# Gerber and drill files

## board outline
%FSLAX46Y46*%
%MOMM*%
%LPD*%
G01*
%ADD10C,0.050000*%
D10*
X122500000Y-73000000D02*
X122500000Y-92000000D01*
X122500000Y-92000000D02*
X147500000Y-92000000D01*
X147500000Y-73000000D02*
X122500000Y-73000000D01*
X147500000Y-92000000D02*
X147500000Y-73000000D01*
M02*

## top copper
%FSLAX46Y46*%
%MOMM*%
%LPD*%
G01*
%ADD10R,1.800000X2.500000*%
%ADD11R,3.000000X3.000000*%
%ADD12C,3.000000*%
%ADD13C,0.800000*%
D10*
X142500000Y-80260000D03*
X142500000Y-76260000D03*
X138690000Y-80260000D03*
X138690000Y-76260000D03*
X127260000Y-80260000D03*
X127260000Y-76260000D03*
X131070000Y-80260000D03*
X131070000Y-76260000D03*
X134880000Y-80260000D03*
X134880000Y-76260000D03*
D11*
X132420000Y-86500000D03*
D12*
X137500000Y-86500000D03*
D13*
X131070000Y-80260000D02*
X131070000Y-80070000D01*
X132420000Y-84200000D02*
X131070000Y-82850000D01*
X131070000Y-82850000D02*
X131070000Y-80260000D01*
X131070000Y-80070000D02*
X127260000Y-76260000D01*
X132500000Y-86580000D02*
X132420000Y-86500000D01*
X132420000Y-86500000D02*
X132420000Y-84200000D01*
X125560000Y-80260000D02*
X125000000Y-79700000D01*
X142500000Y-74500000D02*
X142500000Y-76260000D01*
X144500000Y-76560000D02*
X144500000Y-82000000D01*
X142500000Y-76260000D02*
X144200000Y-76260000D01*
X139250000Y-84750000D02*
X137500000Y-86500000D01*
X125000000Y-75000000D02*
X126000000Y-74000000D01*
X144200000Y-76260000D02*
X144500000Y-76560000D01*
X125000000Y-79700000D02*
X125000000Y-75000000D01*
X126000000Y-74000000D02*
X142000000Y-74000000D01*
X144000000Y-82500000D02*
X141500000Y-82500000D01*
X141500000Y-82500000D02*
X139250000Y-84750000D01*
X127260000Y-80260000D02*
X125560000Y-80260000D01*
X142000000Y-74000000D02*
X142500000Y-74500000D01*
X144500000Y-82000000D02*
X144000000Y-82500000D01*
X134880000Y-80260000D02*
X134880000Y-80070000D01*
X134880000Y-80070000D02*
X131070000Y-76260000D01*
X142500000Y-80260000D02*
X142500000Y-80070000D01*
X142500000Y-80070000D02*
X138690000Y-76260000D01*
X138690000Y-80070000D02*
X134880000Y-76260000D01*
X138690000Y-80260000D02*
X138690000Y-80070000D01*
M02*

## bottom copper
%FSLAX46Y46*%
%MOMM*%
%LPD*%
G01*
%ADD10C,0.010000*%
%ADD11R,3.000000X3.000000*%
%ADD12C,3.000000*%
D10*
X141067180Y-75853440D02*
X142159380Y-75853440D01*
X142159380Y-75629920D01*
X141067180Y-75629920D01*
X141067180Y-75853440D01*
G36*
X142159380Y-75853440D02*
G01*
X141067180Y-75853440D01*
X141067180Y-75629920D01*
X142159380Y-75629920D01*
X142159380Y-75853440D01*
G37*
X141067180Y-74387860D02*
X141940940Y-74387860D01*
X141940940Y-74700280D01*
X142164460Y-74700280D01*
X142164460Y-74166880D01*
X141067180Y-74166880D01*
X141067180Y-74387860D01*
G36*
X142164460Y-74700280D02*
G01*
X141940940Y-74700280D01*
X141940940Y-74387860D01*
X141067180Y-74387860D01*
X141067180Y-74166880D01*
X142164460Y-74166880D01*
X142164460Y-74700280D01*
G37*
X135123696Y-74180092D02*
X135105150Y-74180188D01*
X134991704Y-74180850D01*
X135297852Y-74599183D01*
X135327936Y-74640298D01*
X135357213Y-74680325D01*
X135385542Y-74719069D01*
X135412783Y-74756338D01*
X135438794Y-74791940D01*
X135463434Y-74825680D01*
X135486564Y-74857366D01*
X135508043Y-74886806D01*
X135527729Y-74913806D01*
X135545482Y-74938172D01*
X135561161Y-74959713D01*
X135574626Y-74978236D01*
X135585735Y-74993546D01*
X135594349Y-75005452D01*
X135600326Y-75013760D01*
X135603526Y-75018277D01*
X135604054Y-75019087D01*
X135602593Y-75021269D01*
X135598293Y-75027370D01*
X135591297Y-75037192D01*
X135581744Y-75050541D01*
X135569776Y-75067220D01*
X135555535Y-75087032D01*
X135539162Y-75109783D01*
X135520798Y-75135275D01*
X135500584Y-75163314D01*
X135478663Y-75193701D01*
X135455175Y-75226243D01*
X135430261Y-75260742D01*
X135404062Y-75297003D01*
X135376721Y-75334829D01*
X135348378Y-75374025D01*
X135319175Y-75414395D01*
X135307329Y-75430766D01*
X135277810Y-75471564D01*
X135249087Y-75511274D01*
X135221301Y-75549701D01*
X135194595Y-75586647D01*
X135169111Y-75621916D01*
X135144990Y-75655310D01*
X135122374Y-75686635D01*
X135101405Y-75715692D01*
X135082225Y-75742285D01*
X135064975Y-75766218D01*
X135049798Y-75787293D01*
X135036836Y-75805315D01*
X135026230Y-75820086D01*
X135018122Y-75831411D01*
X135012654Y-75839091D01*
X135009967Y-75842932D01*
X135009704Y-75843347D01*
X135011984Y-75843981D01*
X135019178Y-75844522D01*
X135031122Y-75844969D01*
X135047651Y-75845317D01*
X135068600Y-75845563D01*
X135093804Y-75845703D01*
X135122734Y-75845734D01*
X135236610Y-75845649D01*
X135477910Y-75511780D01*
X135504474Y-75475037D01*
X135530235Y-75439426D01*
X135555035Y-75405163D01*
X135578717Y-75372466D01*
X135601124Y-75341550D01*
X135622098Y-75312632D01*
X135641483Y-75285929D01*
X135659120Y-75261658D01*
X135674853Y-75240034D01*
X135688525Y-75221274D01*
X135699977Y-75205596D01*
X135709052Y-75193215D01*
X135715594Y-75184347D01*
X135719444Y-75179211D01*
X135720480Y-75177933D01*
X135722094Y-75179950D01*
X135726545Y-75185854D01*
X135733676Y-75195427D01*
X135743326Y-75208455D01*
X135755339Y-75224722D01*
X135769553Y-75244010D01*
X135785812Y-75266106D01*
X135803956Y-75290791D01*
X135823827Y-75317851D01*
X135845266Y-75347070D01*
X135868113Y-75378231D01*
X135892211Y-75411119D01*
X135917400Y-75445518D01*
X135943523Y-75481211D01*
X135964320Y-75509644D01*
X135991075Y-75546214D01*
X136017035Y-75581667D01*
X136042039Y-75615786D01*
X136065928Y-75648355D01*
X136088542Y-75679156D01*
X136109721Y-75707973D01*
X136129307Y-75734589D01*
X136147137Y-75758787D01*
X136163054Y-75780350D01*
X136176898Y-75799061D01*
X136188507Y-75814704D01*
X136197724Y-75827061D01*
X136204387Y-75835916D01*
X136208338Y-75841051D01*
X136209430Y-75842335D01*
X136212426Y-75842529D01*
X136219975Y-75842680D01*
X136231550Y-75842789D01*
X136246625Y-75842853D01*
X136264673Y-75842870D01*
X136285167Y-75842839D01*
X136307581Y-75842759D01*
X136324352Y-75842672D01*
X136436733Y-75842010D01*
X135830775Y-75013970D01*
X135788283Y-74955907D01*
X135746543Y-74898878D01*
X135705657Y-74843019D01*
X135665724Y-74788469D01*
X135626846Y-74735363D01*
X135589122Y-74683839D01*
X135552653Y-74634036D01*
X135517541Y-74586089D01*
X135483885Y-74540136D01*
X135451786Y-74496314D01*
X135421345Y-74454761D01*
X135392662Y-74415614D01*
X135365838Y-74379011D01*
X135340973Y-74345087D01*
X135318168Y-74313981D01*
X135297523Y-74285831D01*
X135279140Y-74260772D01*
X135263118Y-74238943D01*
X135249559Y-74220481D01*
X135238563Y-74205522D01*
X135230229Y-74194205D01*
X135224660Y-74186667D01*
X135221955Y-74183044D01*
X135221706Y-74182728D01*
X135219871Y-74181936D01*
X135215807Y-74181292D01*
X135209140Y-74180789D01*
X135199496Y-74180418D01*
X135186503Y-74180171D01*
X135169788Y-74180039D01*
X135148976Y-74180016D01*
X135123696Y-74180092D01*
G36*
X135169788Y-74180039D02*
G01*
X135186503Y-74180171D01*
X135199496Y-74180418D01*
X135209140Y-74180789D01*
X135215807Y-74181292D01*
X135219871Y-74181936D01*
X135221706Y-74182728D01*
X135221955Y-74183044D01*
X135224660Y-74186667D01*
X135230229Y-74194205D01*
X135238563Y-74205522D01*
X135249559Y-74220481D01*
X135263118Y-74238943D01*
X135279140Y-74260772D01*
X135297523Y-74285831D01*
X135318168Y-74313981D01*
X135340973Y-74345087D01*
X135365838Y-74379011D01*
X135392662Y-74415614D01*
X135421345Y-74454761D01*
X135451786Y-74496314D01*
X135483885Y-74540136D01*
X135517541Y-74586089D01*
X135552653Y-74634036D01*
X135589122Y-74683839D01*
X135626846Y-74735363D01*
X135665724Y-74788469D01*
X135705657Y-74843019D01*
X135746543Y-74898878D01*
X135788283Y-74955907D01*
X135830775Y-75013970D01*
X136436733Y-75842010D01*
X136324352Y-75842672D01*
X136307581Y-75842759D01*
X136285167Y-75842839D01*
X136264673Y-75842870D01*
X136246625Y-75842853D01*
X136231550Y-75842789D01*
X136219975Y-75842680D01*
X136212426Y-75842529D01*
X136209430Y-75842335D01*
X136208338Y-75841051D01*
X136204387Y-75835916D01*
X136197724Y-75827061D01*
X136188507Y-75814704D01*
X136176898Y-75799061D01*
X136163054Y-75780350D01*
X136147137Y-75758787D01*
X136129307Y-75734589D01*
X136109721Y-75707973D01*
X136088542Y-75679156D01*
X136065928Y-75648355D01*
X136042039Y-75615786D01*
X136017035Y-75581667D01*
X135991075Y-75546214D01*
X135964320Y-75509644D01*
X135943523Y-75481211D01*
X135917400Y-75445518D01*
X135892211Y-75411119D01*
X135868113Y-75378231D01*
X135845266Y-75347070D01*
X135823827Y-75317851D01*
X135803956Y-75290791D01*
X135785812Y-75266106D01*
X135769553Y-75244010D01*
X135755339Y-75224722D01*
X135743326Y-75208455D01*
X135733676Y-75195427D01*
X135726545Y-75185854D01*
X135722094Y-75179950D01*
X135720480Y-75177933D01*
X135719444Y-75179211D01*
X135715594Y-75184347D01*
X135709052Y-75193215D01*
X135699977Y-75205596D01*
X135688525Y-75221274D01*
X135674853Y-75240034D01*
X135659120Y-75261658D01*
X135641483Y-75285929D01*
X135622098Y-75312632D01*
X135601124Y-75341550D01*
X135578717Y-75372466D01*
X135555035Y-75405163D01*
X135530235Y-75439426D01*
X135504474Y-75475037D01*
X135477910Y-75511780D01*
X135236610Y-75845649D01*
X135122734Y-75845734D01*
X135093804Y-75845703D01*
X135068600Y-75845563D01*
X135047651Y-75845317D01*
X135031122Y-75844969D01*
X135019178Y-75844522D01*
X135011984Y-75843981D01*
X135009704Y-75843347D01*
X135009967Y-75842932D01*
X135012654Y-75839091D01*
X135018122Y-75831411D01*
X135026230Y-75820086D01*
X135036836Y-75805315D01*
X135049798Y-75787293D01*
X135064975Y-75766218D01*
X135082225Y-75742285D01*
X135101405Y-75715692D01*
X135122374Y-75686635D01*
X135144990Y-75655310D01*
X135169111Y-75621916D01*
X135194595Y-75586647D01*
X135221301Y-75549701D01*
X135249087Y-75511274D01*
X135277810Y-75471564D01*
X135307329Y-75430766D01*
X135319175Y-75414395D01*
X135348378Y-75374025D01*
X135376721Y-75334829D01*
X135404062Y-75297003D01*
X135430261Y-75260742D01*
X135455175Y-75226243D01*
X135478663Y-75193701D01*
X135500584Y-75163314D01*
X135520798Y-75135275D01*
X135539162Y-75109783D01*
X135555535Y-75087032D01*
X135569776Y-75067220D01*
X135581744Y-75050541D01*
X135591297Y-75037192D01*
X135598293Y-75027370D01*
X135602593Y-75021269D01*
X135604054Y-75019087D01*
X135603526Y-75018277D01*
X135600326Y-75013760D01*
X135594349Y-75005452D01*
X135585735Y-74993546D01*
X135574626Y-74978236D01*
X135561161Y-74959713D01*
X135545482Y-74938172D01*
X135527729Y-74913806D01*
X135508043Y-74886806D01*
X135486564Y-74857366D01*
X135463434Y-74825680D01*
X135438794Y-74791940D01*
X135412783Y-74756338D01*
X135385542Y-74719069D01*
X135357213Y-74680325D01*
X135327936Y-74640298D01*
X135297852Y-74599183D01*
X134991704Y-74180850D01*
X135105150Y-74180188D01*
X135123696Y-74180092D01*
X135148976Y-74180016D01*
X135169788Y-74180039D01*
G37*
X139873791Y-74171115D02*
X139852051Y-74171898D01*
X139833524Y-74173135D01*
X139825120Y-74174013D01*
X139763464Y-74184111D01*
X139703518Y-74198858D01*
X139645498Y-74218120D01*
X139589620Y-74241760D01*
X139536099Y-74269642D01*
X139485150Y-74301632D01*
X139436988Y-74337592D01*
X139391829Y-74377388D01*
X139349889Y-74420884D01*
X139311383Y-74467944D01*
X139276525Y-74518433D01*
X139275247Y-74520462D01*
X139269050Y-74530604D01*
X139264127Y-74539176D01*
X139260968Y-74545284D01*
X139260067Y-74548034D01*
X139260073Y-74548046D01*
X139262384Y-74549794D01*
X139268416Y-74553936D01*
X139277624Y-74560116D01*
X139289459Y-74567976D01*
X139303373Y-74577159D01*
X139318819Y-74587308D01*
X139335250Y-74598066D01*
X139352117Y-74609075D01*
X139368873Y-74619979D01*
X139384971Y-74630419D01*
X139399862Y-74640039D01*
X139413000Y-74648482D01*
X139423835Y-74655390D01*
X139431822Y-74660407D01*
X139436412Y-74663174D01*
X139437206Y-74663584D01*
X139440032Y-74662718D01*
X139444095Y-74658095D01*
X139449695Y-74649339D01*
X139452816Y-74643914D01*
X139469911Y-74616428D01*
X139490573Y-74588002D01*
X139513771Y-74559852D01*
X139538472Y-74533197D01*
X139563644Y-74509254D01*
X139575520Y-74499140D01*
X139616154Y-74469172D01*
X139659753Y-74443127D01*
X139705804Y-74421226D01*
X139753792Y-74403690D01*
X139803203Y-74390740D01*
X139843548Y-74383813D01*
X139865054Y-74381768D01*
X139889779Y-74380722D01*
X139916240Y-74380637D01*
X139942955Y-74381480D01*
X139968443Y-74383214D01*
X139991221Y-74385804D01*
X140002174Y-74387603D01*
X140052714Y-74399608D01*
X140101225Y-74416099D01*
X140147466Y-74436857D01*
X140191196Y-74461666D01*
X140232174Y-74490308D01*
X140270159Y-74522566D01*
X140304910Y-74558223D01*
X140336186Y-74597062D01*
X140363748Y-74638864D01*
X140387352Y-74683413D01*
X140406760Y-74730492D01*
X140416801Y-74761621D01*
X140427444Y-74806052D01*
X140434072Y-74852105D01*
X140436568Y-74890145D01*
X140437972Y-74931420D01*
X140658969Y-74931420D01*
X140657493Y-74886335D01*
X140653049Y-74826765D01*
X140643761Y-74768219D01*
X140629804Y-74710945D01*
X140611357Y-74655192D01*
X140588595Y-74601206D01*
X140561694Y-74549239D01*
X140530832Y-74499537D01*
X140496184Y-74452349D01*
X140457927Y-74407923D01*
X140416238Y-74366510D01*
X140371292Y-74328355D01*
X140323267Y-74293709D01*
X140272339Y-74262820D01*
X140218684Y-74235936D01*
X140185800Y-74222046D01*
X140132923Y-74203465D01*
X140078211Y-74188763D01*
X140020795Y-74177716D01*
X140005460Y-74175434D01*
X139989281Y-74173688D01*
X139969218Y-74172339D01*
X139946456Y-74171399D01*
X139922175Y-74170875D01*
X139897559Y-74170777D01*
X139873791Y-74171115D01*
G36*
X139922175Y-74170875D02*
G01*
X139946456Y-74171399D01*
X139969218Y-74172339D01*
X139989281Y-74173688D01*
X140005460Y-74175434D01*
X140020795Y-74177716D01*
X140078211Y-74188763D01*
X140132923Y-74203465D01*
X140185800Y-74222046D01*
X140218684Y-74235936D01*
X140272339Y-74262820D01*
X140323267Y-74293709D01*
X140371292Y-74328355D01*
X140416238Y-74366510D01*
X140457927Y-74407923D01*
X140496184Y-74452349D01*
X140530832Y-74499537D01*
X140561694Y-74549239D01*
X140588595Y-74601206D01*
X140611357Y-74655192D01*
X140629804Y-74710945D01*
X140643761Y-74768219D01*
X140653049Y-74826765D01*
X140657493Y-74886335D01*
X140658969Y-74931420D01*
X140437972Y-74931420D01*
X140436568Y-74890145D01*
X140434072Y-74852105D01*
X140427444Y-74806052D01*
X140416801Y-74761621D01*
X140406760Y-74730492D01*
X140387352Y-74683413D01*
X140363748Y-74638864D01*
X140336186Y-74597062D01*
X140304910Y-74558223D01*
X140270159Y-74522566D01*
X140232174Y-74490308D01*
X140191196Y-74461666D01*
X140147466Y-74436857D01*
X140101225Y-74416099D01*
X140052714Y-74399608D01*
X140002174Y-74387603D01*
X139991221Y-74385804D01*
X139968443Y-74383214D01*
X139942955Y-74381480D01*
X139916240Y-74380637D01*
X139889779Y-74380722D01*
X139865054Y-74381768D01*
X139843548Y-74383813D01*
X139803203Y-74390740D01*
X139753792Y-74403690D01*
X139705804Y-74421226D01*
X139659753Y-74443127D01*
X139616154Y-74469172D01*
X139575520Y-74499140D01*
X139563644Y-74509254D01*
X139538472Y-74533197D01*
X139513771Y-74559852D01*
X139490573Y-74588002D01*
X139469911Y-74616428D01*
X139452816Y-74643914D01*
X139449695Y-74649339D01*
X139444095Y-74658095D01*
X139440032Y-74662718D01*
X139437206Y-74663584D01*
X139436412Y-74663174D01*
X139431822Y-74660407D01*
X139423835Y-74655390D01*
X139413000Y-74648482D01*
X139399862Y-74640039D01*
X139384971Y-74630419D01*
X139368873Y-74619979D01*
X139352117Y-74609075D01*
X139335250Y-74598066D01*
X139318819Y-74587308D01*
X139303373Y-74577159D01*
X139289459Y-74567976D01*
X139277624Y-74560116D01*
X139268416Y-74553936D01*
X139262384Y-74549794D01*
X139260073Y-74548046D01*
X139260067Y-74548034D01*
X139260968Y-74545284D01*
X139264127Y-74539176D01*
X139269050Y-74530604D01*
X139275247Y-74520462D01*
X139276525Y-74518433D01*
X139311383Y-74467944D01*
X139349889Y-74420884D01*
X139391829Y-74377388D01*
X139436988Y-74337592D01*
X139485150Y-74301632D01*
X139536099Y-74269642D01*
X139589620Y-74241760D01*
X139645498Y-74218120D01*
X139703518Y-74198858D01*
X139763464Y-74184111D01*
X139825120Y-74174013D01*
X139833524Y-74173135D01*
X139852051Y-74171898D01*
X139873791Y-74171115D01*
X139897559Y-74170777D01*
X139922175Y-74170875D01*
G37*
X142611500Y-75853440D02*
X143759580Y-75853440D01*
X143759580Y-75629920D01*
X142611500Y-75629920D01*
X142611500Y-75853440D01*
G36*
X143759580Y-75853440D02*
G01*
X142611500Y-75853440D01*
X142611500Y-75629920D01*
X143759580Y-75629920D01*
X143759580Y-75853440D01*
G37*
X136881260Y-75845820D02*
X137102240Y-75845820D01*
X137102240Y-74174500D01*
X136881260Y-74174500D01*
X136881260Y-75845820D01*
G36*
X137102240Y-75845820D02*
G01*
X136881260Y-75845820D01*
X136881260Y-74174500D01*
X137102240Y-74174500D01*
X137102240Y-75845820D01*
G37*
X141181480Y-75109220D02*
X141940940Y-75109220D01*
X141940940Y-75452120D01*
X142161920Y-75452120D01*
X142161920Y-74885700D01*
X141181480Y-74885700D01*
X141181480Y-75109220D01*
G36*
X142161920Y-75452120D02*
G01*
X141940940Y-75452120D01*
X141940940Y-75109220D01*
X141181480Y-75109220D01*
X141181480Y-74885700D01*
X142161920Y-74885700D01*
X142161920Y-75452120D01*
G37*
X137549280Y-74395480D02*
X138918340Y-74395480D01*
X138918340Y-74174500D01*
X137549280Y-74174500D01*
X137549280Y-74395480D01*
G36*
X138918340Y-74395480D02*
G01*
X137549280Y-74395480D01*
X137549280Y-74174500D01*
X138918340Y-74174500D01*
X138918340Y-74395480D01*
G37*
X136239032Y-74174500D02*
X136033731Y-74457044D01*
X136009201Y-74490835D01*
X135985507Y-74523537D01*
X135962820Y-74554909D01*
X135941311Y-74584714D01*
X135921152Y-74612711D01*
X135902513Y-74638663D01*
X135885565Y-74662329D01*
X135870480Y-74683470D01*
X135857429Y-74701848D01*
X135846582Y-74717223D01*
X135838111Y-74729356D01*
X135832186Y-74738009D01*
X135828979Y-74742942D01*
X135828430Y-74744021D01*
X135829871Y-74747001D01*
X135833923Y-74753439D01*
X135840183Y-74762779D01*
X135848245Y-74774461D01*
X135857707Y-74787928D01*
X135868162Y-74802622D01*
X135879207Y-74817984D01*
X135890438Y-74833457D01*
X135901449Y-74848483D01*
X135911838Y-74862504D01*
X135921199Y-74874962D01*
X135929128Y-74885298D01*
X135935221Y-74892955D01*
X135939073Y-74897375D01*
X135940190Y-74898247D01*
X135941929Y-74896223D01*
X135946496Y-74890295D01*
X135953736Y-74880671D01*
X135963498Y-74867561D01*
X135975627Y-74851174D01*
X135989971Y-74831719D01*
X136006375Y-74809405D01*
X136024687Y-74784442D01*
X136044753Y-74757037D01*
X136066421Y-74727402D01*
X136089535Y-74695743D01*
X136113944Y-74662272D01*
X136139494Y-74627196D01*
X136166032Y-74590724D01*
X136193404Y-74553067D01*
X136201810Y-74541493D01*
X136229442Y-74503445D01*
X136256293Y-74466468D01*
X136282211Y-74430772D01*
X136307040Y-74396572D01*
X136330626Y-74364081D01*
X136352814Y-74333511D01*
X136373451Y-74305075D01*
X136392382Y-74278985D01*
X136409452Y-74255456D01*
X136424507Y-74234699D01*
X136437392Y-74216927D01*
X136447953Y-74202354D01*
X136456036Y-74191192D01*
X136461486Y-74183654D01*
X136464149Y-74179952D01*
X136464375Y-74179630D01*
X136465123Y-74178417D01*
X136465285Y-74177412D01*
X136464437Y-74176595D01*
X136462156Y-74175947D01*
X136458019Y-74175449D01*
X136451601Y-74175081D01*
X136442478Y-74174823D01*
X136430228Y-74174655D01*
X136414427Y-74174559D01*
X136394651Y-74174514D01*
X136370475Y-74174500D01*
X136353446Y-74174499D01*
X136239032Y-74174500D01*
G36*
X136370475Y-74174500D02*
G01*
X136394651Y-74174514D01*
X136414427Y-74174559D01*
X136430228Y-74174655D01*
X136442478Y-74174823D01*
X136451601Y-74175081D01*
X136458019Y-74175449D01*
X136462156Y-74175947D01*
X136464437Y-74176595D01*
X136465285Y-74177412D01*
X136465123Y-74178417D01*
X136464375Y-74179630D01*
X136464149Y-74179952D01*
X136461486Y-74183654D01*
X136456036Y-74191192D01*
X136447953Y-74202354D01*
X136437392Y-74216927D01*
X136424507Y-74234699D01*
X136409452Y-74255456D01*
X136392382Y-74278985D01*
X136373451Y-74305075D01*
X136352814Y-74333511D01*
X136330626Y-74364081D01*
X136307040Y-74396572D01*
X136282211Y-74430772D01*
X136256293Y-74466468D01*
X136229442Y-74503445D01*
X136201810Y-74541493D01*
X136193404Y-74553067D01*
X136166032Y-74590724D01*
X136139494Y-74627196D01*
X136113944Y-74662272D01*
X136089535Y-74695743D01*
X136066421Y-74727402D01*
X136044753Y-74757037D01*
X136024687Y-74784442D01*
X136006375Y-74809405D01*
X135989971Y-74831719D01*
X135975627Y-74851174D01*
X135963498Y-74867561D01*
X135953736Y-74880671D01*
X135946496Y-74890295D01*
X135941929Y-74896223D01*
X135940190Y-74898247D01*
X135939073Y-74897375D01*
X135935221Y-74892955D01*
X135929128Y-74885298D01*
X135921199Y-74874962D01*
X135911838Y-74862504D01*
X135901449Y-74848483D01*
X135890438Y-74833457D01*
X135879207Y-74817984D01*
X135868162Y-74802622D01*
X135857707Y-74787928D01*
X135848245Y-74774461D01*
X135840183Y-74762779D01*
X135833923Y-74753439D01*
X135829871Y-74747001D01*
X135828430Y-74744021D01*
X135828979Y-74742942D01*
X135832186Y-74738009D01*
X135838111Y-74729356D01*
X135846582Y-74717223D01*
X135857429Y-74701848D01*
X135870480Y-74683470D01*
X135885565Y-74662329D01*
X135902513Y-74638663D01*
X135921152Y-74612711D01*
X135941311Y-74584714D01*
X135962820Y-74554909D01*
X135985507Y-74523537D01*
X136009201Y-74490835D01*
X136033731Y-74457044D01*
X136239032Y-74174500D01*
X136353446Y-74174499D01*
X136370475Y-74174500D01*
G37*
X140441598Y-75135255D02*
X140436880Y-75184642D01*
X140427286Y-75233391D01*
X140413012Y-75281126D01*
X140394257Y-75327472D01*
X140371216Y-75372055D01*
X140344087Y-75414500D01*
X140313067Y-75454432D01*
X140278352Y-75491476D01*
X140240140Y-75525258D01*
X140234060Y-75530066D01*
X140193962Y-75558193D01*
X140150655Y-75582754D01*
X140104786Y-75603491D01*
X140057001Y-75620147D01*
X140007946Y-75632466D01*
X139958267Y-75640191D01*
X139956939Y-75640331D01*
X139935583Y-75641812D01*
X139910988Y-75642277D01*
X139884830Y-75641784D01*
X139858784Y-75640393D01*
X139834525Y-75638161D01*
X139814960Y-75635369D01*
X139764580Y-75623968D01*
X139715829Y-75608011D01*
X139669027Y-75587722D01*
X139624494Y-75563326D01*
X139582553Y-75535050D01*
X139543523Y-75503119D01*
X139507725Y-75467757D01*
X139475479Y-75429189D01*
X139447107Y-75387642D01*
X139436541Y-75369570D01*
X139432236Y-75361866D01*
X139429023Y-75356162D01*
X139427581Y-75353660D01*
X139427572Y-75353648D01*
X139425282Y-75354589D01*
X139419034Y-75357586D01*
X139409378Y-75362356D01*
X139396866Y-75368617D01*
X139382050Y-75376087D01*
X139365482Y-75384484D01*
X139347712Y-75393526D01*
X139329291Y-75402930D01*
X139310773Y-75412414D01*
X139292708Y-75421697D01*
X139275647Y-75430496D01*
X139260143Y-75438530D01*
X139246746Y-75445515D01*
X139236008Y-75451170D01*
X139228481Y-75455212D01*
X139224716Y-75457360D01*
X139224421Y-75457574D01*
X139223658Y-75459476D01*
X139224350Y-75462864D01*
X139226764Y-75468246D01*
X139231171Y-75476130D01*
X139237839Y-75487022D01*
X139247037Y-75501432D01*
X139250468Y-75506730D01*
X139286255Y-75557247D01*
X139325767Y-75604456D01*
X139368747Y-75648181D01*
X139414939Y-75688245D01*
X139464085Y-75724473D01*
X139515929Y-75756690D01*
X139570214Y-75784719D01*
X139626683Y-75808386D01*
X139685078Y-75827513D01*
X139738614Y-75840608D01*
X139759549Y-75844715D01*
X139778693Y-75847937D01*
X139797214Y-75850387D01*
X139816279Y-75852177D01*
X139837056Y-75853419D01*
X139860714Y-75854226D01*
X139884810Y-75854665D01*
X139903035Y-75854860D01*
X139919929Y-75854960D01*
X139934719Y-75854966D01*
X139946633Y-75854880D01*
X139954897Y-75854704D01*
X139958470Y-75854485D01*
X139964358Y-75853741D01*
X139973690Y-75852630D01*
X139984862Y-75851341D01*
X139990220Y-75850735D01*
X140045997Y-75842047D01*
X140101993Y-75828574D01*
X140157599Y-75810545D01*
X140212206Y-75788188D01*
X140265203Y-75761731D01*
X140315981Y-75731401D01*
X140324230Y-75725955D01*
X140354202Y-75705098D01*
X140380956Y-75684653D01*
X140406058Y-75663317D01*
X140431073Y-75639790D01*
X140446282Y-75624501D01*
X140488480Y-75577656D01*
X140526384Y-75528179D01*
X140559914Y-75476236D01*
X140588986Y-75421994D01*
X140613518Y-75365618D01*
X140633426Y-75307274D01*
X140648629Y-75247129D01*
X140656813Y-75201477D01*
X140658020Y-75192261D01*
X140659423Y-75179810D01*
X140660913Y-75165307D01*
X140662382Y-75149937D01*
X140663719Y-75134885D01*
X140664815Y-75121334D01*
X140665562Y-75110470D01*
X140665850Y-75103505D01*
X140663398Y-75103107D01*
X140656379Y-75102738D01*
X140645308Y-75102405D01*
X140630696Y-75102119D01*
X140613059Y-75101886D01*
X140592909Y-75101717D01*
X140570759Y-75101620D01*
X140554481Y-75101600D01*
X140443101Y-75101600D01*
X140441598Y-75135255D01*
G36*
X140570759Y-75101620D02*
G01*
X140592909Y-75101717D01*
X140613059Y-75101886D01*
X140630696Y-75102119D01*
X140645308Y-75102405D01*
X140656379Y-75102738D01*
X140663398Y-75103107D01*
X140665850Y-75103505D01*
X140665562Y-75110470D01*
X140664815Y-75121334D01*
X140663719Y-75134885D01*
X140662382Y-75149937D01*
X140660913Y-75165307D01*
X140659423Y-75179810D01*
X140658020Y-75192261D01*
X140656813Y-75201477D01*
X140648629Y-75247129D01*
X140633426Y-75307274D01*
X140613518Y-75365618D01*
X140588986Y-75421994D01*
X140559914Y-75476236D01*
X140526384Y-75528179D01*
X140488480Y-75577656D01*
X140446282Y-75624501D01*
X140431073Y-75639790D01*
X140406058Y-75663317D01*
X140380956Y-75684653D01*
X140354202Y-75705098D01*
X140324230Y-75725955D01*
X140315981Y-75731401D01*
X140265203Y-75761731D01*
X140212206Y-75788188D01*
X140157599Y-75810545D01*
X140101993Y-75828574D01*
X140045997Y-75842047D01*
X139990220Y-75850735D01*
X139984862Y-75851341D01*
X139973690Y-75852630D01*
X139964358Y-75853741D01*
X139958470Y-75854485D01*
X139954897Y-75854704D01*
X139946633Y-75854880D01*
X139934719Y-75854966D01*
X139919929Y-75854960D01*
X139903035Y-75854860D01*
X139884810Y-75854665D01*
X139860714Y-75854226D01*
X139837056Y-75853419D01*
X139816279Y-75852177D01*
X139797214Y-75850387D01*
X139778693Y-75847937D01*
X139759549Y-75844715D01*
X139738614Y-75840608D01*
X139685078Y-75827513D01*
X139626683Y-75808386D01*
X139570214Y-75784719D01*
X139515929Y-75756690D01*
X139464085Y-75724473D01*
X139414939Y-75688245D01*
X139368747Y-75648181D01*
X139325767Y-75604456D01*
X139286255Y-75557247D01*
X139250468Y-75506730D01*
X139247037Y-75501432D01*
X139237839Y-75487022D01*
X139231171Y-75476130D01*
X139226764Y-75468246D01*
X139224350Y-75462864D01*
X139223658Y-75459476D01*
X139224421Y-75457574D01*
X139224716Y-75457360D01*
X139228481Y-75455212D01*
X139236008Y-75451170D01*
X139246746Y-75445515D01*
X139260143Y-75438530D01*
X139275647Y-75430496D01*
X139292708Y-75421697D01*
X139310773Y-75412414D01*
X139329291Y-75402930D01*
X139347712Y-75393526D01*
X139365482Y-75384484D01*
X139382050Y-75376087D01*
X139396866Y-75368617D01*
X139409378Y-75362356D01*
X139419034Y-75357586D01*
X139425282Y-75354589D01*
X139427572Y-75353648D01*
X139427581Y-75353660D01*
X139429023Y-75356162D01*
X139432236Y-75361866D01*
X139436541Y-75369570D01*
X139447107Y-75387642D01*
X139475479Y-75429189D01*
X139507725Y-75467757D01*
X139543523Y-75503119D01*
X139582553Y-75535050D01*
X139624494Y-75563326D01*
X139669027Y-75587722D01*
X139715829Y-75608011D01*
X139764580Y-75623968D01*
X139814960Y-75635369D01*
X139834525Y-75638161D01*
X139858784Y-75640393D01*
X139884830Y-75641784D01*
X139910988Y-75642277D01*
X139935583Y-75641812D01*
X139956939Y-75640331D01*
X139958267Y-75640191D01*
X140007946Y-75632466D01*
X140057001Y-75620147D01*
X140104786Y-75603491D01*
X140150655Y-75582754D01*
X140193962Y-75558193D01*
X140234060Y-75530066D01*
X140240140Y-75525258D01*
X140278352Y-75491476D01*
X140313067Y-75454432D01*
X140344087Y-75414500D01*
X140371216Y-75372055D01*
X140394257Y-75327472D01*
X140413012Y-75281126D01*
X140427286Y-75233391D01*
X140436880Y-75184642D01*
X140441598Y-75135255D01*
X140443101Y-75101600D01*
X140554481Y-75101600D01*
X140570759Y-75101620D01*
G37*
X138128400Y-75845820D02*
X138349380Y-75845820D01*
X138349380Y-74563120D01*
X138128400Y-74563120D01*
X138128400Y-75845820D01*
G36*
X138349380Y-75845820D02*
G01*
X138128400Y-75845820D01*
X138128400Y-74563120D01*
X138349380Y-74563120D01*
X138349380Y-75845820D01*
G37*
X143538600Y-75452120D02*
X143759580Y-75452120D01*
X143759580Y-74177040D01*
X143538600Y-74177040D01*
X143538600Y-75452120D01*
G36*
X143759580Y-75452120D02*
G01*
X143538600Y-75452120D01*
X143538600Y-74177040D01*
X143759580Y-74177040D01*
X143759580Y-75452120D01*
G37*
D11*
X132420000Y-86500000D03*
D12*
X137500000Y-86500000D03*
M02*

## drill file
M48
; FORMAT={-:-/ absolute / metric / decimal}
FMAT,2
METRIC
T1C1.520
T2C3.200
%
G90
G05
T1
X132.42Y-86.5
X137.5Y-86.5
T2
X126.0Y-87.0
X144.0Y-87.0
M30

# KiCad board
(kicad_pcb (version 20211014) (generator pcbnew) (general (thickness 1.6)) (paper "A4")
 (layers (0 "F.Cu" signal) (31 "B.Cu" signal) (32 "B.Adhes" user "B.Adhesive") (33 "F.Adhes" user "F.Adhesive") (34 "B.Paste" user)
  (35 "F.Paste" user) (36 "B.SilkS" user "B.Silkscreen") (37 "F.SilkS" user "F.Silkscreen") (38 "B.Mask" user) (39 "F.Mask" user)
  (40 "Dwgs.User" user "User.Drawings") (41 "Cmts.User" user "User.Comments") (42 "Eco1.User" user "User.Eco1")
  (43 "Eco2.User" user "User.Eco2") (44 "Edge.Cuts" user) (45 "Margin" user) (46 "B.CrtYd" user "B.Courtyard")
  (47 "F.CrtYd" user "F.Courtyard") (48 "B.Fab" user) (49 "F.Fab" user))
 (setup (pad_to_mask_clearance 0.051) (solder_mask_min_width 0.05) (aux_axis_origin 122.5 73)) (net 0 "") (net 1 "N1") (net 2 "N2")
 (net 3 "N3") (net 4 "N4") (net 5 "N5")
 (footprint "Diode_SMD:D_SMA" (layer "F.Cu") (at 142.5 78.26 90)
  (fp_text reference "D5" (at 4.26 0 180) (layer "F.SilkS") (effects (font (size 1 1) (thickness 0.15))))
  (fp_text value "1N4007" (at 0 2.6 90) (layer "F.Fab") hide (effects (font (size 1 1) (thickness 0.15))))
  (pad "1" smd rect locked (at -2 0 90) (size 2.5 1.8) (layers "F.Cu" "F.Paste" "F.Mask") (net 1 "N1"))
  (pad "2" smd rect locked (at 2 0 90) (size 2.5 1.8) (layers "F.Cu" "F.Paste" "F.Mask") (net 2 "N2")))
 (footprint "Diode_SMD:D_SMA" (layer "F.Cu") (at 138.69 78.26 90)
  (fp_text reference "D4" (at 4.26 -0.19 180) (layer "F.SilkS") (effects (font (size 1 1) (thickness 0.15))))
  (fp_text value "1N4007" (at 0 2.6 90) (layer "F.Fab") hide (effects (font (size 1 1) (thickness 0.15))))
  (pad "1" smd rect locked (at -2 0 90) (size 2.5 1.8) (layers "F.Cu" "F.Paste" "F.Mask") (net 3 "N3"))
  (pad "2" smd rect locked (at 2 0 90) (size 2.5 1.8) (layers "F.Cu" "F.Paste" "F.Mask") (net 1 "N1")))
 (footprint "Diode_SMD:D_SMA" (layer "F.Cu") (at 127.26 78.26 90)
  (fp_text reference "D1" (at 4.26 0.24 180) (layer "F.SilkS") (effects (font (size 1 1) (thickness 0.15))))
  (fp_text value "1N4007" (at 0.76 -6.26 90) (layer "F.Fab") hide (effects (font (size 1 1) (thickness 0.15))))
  (pad "1" smd rect locked (at -2 0 90) (size 2.5 1.8) (layers "F.Cu" "F.Paste" "F.Mask") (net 2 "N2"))
  (pad "2" smd rect locked (at 2 0 90) (size 2.5 1.8) (layers "F.Cu" "F.Paste" "F.Mask") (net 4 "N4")))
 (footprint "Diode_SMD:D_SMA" (layer "F.Cu") (at 131.07 78.26 90)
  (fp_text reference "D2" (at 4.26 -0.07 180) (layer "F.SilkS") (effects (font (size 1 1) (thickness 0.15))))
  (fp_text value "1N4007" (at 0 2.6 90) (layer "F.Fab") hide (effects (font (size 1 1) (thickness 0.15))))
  (pad "1" smd rect locked (at -2 0 90) (size 2.5 1.8) (layers "F.Cu" "F.Paste" "F.Mask") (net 4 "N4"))
  (pad "2" smd rect locked (at 2 0 90) (size 2.5 1.8) (layers "F.Cu" "F.Paste" "F.Mask") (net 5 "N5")))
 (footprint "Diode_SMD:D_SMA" (layer "F.Cu") (at 134.88 78.26 90)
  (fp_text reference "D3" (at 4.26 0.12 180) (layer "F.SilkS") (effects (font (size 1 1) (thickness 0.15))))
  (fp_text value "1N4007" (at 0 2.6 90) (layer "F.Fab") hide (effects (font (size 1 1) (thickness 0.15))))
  (pad "1" smd rect locked (at -2 0 90) (size 2.5 1.8) (layers "F.Cu" "F.Paste" "F.Mask") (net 5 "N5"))
  (pad "2" smd rect locked (at 2 0 90) (size 2.5 1.8) (layers "F.Cu" "F.Paste" "F.Mask") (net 3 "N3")))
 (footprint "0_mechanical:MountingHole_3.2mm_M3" (layer "F.Cu") (at 144 87)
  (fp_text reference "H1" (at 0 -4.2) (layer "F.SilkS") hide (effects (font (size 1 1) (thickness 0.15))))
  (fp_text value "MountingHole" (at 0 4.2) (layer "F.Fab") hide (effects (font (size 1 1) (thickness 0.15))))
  (pad "" np_thru_hole circle locked (at 0 0) (size 3.2 3.2) (drill 3.2) (layers *.Cu *.Mask)))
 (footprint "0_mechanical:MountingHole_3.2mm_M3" (layer "F.Cu") (at 126 87)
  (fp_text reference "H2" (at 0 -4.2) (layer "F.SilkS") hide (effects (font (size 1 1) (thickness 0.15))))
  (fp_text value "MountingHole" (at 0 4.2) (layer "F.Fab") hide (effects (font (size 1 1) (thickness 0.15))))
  (pad "" np_thru_hole circle locked (at 0 0) (size 3.2 3.2) (drill 3.2) (layers *.Cu *.Mask)))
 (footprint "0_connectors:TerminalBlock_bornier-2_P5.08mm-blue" (layer "F.Cu") (at 132.42 86.5)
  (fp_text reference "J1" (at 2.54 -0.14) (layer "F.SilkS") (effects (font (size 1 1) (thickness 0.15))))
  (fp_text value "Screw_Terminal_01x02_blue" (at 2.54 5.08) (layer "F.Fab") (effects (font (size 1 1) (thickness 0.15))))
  (pad "1" thru_hole rect locked (at 0 0) (size 3 3) (drill 1.52) (layers *.Cu *.Mask) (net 4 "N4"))
  (pad "2" thru_hole circle locked (at 5.08 0) (size 3 3) (drill 1.52) (layers *.Cu *.Mask) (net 2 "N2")))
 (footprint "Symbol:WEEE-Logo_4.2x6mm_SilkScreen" (layer "B.Cu") (at 130 80.5 180)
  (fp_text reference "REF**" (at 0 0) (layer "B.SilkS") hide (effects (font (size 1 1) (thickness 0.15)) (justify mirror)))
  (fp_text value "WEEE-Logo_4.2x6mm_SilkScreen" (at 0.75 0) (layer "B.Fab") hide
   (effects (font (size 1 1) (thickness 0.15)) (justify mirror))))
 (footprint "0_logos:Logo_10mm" (layer "B.Cu") (at 139.5 75 180)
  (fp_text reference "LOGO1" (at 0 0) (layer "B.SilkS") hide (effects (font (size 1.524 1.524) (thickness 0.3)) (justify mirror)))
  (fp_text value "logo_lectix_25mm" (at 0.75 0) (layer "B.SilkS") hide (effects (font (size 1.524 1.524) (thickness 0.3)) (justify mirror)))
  (fp_poly
   (pts (xy -1.56718 -0.85344) (xy -2.65938 -0.85344) (xy -2.65938 -0.62992) (xy -1.56718 -0.62992) (xy -1.56718 -0.85344)) (layer "B.Cu")
   (width 0.01) (fill solid))
  (fp_poly
   (pts (xy -1.56718 0.61214) (xy -2.44094 0.61214) (xy -2.44094 0.29972) (xy -2.66446 0.29972) (xy -2.66446 0.83312) (xy -1.56718 0.83312)
    (xy -1.56718 0.61214))
   (layer "B.Cu") (width 0.01) (fill solid))
  (fp_poly
   (pts (xy 4.376304 0.819908) (xy 4.39485 0.819812) (xy 4.508296 0.81915) (xy 4.202148 0.400817) (xy 4.172064 0.359702)
    (xy 4.142787 0.319675) (xy 4.114458 0.280931) (xy 4.087217 0.243662) (xy 4.061206 0.20806) (xy 4.036566 0.17432) (xy 4.013436 0.142634)
    (xy 3.991957 0.113194) (xy 3.972271 0.086194) (xy 3.954518 0.061828) (xy 3.938839 0.040287) (xy 3.925374 0.021764)
    (xy 3.914265 0.006454) (xy 3.905651 -0.005452) (xy 3.899674 -0.01376) (xy 3.896474 -0.018277) (xy 3.895946 -0.019087)
    (xy 3.897407 -0.021269) (xy 3.901707 -0.02737) (xy 3.908703 -0.037192) (xy 3.918256 -0.050541) (xy 3.930224 -0.06722)
    (xy 3.944465 -0.087032) (xy 3.960838 -0.109783) (xy 3.979202 -0.135275) (xy 3.999416 -0.163314) (xy 4.021337 -0.193701)
    (xy 4.044825 -0.226243) (xy 4.069739 -0.260742) (xy 4.095938 -0.297003) (xy 4.123279 -0.334829) (xy 4.151622 -0.374025)
    (xy 4.180825 -0.414395) (xy 4.192671 -0.430766) (xy 4.22219 -0.471564) (xy 4.250913 -0.511274) (xy 4.278699 -0.549701)
    (xy 4.305405 -0.586647) (xy 4.330889 -0.621916) (xy 4.35501 -0.65531) (xy 4.377626 -0.686635) (xy 4.398595 -0.715692)
    (xy 4.417775 -0.742285) (xy 4.435025 -0.766218) (xy 4.450202 -0.787293) (xy 4.463164 -0.805315) (xy 4.47377 -0.820086)
    (xy 4.481878 -0.831411) (xy 4.487346 -0.839091) (xy 4.490033 -0.842932) (xy 4.490296 -0.843347) (xy 4.488016 -0.843981)
    (xy 4.480822 -0.844522) (xy 4.468878 -0.844969) (xy 4.452349 -0.845317) (xy 4.4314 -0.845563) (xy 4.406196 -0.845703)
    (xy 4.377266 -0.845734) (xy 4.26339 -0.845649) (xy 4.02209 -0.51178) (xy 3.995526 -0.475037) (xy 3.969765 -0.439426)
    (xy 3.944965 -0.405163) (xy 3.921283 -0.372466) (xy 3.898876 -0.34155) (xy 3.877902 -0.312632) (xy 3.858517 -0.285929)
    (xy 3.84088 -0.261658) (xy 3.825147 -0.240034) (xy 3.811475 -0.221274) (xy 3.800023 -0.205596) (xy 3.790948 -0.193215)
    (xy 3.784406 -0.184347) (xy 3.780556 -0.179211) (xy 3.77952 -0.177933) (xy 3.777906 -0.17995) (xy 3.773455 -0.185854)
    (xy 3.766324 -0.195427) (xy 3.756674 -0.208455) (xy 3.744661 -0.224722) (xy 3.730447 -0.24401) (xy 3.714188 -0.266106)
    (xy 3.696044 -0.290791) (xy 3.676173 -0.317851) (xy 3.654734 -0.34707) (xy 3.631887 -0.378231) (xy 3.607789 -0.411119)
    (xy 3.5826 -0.445518) (xy 3.556477 -0.481211) (xy 3.53568 -0.509644) (xy 3.508925 -0.546214) (xy 3.482965 -0.581667)
    (xy 3.457961 -0.615786) (xy 3.434072 -0.648355) (xy 3.411458 -0.679156) (xy 3.390279 -0.707973) (xy 3.370693 -0.734589)
    (xy 3.352863 -0.758787) (xy 3.336946 -0.78035) (xy 3.323102 -0.799061) (xy 3.311493 -0.814704) (xy 3.302276 -0.827061)
    (xy 3.295613 -0.835916) (xy 3.291662 -0.841051) (xy 3.29057 -0.842335) (xy 3.287574 -0.842529) (xy 3.280025 -0.84268)
    (xy 3.26845 -0.842789) (xy 3.253375 -0.842853) (xy 3.235327 -0.84287) (xy 3.214833 -0.842839) (xy 3.192419 -0.842759)
    (xy 3.175648 -0.842672) (xy 3.063267 -0.84201) (xy 3.669225 -0.01397) (xy 3.711717 0.044093) (xy 3.753457 0.101122)
    (xy 3.794343 0.156981) (xy 3.834276 0.211531) (xy 3.873154 0.264637) (xy 3.910878 0.316161) (xy 3.947347 0.365964)
    (xy 3.982459 0.413911) (xy 4.016115 0.459864) (xy 4.048214 0.503686) (xy 4.078655 0.545239) (xy 4.107338 0.584386)
    (xy 4.134162 0.620989) (xy 4.159027 0.654913) (xy 4.181832 0.686019) (xy 4.202477 0.714169) (xy 4.22086 0.739228) (xy 4.236882 0.761057)
    (xy 4.250441 0.779519) (xy 4.261437 0.794478) (xy 4.269771 0.805795) (xy 4.27534 0.813333) (xy 4.278045 0.816956) (xy 4.278294 0.817272)
    (xy 4.280129 0.818064) (xy 4.284193 0.818708) (xy 4.29086 0.819211) (xy 4.300504 0.819582) (xy 4.313497 0.819829) (xy 4.330212 0.819961)
    (xy 4.351024 0.819984) (xy 4.376304 0.819908))
   (layer "B.Cu") (width 0.01) (fill solid))
  (fp_poly
   (pts (xy -0.373791 0.828885) (xy -0.352051 0.828102) (xy -0.333524 0.826865) (xy -0.32512 0.825987) (xy -0.263464 0.815889)
    (xy -0.203518 0.801142) (xy -0.145498 0.78188) (xy -0.08962 0.75824) (xy -0.036099 0.730358) (xy 0.01485 0.698368)
    (xy 0.063012 0.662408) (xy 0.108171 0.622612) (xy 0.150111 0.579116) (xy 0.188617 0.532056) (xy 0.223475 0.481567)
    (xy 0.224753 0.479538) (xy 0.23095 0.469396) (xy 0.235873 0.460824) (xy 0.239032 0.454716) (xy 0.239933 0.451966) (xy 0.239927 0.451954)
    (xy 0.237616 0.450206) (xy 0.231584 0.446064) (xy 0.222376 0.439884) (xy 0.210541 0.432024) (xy 0.196627 0.422841)
    (xy 0.181181 0.412692) (xy 0.16475 0.401934) (xy 0.147883 0.390925) (xy 0.131127 0.380021) (xy 0.115029 0.369581) (xy 0.100138 0.359961)
    (xy 0.087 0.351518) (xy 0.076165 0.34461) (xy 0.068178 0.339593) (xy 0.063588 0.336826) (xy 0.062794 0.336416) (xy 0.059968 0.337282)
    (xy 0.055905 0.341905) (xy 0.050305 0.350661) (xy 0.047184 0.356086) (xy 0.030089 0.383572) (xy 0.009427 0.411998)
    (xy -0.013771 0.440148) (xy -0.038472 0.466803) (xy -0.063644 0.490746) (xy -0.07552 0.50086) (xy -0.116154 0.530828)
    (xy -0.159753 0.556873) (xy -0.205804 0.578774) (xy -0.253792 0.59631) (xy -0.303203 0.60926) (xy -0.343548 0.616187)
    (xy -0.365054 0.618232) (xy -0.389779 0.619278) (xy -0.41624 0.619363) (xy -0.442955 0.61852) (xy -0.468443 0.616786)
    (xy -0.491221 0.614196) (xy -0.502174 0.612397) (xy -0.552714 0.600392) (xy -0.601225 0.583901) (xy -0.647466 0.563143)
    (xy -0.691196 0.538334) (xy -0.732174 0.509692) (xy -0.770159 0.477434) (xy -0.80491 0.441777) (xy -0.836186 0.402938)
    (xy -0.863748 0.361136) (xy -0.887352 0.316587) (xy -0.90676 0.269508) (xy -0.916801 0.238379) (xy -0.927444 0.193948)
    (xy -0.934072 0.147895) (xy -0.936568 0.109855) (xy -0.937972 0.06858) (xy -1.158969 0.06858) (xy -1.157493 0.113665)
    (xy -1.153049 0.173235) (xy -1.143761 0.231781) (xy -1.129804 0.289055) (xy -1.111357 0.344808) (xy -1.088595 0.398794)
    (xy -1.061694 0.450761) (xy -1.030832 0.500463) (xy -0.996184 0.547651) (xy -0.957927 0.592077) (xy -0.916238 0.63349)
    (xy -0.871292 0.671645) (xy -0.823267 0.706291) (xy -0.772339 0.73718) (xy -0.718684 0.764064) (xy -0.6858 0.777954)
    (xy -0.632923 0.796535) (xy -0.578211 0.811237) (xy -0.520795 0.822284) (xy -0.50546 0.824566) (xy -0.489281 0.826312)
    (xy -0.469218 0.827661) (xy -0.446456 0.828601) (xy -0.422175 0.829125) (xy -0.397559 0.829223) (xy -0.373791 0.828885))
   (layer "B.Cu") (width 0.01) (fill solid))
  (fp_poly
   (pts (xy -3.1115 -0.85344) (xy -4.25958 -0.85344) (xy -4.25958 -0.62992) (xy -3.1115 -0.62992) (xy -3.1115 -0.85344)) (layer "B.Cu")
   (width 0.01) (fill solid))
  (fp_poly
   (pts (xy 2.61874 -0.84582) (xy 2.39776 -0.84582) (xy 2.39776 0.8255) (xy 2.61874 0.8255) (xy 2.61874 -0.84582)) (layer "B.Cu")
   (width 0.01) (fill solid))
  (fp_poly
   (pts (xy -1.68148 -0.10922) (xy -2.44094 -0.10922) (xy -2.44094 -0.45212) (xy -2.66192 -0.45212) (xy -2.66192 0.1143)
    (xy -1.68148 0.1143) (xy -1.68148 -0.10922))
   (layer "B.Cu") (width 0.01) (fill solid))
  (fp_poly
   (pts (xy 1.95072 0.60452) (xy 0.58166 0.60452) (xy 0.58166 0.8255) (xy 1.95072 0.8255) (xy 1.95072 0.60452)) (layer "B.Cu") (width 0.01)
   (fill solid))
  (fp_poly
   (pts (xy 3.260968 0.8255) (xy 3.466269 0.542956) (xy 3.490799 0.509165) (xy 3.514493 0.476463) (xy 3.53718 0.445091)
    (xy 3.558689 0.415286) (xy 3.578848 0.387289) (xy 3.597487 0.361337) (xy 3.614435 0.337671) (xy 3.62952 0.31653) (xy 3.642571 0.298152)
    (xy 3.653418 0.282777) (xy 3.661889 0.270644) (xy 3.667814 0.261991) (xy 3.671021 0.257058) (xy 3.67157 0.255979) (xy 3.670129 0.252999)
    (xy 3.666077 0.246561) (xy 3.659817 0.237221) (xy 3.651755 0.225539) (xy 3.642293 0.212072) (xy 3.631838 0.197378)
    (xy 3.620793 0.182016) (xy 3.609562 0.166543) (xy 3.598551 0.151517) (xy 3.588162 0.137496) (xy 3.578801 0.125038)
    (xy 3.570872 0.114702) (xy 3.564779 0.107045) (xy 3.560927 0.102625) (xy 3.55981 0.101753) (xy 3.558071 0.103777) (xy 3.553504 0.109705)
    (xy 3.546264 0.119329) (xy 3.536502 0.132439) (xy 3.524373 0.148826) (xy 3.510029 0.168281) (xy 3.493625 0.190595)
    (xy 3.475313 0.215558) (xy 3.455247 0.242963) (xy 3.433579 0.272598) (xy 3.410465 0.304257) (xy 3.386056 0.337728)
    (xy 3.360506 0.372804) (xy 3.333968 0.409276) (xy 3.306596 0.446933) (xy 3.29819 0.458507) (xy 3.270558 0.496555) (xy 3.243707 0.533532)
    (xy 3.217789 0.569228) (xy 3.19296 0.603428) (xy 3.169374 0.635919) (xy 3.147186 0.666489) (xy 3.126549 0.694925) (xy 3.107618 0.721015)
    (xy 3.090548 0.744544) (xy 3.075493 0.765301) (xy 3.062608 0.783073) (xy 3.052047 0.797646) (xy 3.043964 0.808808)
    (xy 3.038514 0.816346) (xy 3.035851 0.820048) (xy 3.035625 0.82037) (xy 3.034877 0.821583) (xy 3.034715 0.822588) (xy 3.035563 0.823405)
    (xy 3.037844 0.824053) (xy 3.041981 0.824551) (xy 3.048399 0.824919) (xy 3.057522 0.825177) (xy 3.069772 0.825345)
    (xy 3.085573 0.825441) (xy 3.105349 0.825486) (xy 3.129525 0.8255) (xy 3.146554 0.825501) (xy 3.260968 0.8255))
   (layer "B.Cu") (width 0.01) (fill solid))
  (fp_poly
   (pts (xy -0.941598 -0.135255) (xy -0.93688 -0.184642) (xy -0.927286 -0.233391) (xy -0.913012 -0.281126) (xy -0.894257 -0.327472)
    (xy -0.871216 -0.372055) (xy -0.844087 -0.4145) (xy -0.813067 -0.454432) (xy -0.778352 -0.491476) (xy -0.74014 -0.525258)
    (xy -0.73406 -0.530066) (xy -0.693962 -0.558193) (xy -0.650655 -0.582754) (xy -0.604786 -0.603491) (xy -0.557001 -0.620147)
    (xy -0.507946 -0.632466) (xy -0.458267 -0.640191) (xy -0.456939 -0.640331) (xy -0.435583 -0.641812) (xy -0.410988 -0.642277)
    (xy -0.38483 -0.641784) (xy -0.358784 -0.640393) (xy -0.334525 -0.638161) (xy -0.31496 -0.635369) (xy -0.26458 -0.623968)
    (xy -0.215829 -0.608011) (xy -0.169027 -0.587722) (xy -0.124494 -0.563326) (xy -0.082553 -0.53505) (xy -0.043523 -0.503119)
    (xy -0.007725 -0.467757) (xy 0.024521 -0.429189) (xy 0.052893 -0.387642) (xy 0.063459 -0.36957) (xy 0.067764 -0.361866)
    (xy 0.070977 -0.356162) (xy 0.072419 -0.35366) (xy 0.072428 -0.353648) (xy 0.074718 -0.354589) (xy 0.080966 -0.357586)
    (xy 0.090622 -0.362356) (xy 0.103134 -0.368617) (xy 0.11795 -0.376087) (xy 0.134518 -0.384484) (xy 0.152288 -0.393526)
    (xy 0.170709 -0.40293) (xy 0.189227 -0.412414) (xy 0.207292 -0.421697) (xy 0.224353 -0.430496) (xy 0.239857 -0.43853)
    (xy 0.253254 -0.445515) (xy 0.263992 -0.45117) (xy 0.271519 -0.455212) (xy 0.275284 -0.45736) (xy 0.275579 -0.457574)
    (xy 0.276342 -0.459476) (xy 0.27565 -0.462864) (xy 0.273236 -0.468246) (xy 0.268829 -0.47613) (xy 0.262161 -0.487022)
    (xy 0.252963 -0.501432) (xy 0.249532 -0.50673) (xy 0.213745 -0.557247) (xy 0.174233 -0.604456) (xy 0.131253 -0.648181)
    (xy 0.085061 -0.688245) (xy 0.035915 -0.724473) (xy -0.015929 -0.75669) (xy -0.070214 -0.784719) (xy -0.126683 -0.808386)
    (xy -0.185078 -0.827513) (xy -0.238614 -0.840608) (xy -0.259549 -0.844715) (xy -0.278693 -0.847937) (xy -0.297214 -0.850387)
    (xy -0.316279 -0.852177) (xy -0.337056 -0.853419) (xy -0.360714 -0.854226) (xy -0.38481 -0.854665) (xy -0.403035 -0.85486)
    (xy -0.419929 -0.85496) (xy -0.434719 -0.854966) (xy -0.446633 -0.85488) (xy -0.454897 -0.854704) (xy -0.45847 -0.854485)
    (xy -0.464358 -0.853741) (xy -0.47369 -0.85263) (xy -0.484862 -0.851341) (xy -0.49022 -0.850735) (xy -0.545997 -0.842047)
    (xy -0.601993 -0.828574) (xy -0.657599 -0.810545) (xy -0.712206 -0.788188) (xy -0.765203 -0.761731) (xy -0.815981 -0.731401)
    (xy -0.82423 -0.725955) (xy -0.854202 -0.705098) (xy -0.880956 -0.684653) (xy -0.906058 -0.663317) (xy -0.931073 -0.63979)
    (xy -0.946282 -0.624501) (xy -0.98848 -0.577656) (xy -1.026384 -0.528179) (xy -1.059914 -0.476236) (xy -1.088986 -0.421994)
    (xy -1.113518 -0.365618) (xy -1.133426 -0.307274) (xy -1.148629 -0.247129) (xy -1.156813 -0.201477) (xy -1.15802 -0.192261)
    (xy -1.159423 -0.17981) (xy -1.160913 -0.165307) (xy -1.162382 -0.149937) (xy -1.163719 -0.134885) (xy -1.164815 -0.121334)
    (xy -1.165562 -0.11047) (xy -1.16585 -0.103505) (xy -1.163398 -0.103107) (xy -1.156379 -0.102738) (xy -1.145308 -0.102405)
    (xy -1.130696 -0.102119) (xy -1.113059 -0.101886) (xy -1.092909 -0.101717) (xy -1.070759 -0.10162) (xy -1.054481 -0.1016)
    (xy -0.943101 -0.1016) (xy -0.941598 -0.135255))
   (layer "B.Cu") (width 0.01) (fill solid))
  (fp_poly
   (pts (xy 1.3716 -0.84582) (xy 1.15062 -0.84582) (xy 1.15062 0.43688) (xy 1.3716 0.43688) (xy 1.3716 -0.84582)) (layer "B.Cu")
   (width 0.01) (fill solid))
  (fp_poly
   (pts (xy -4.0386 -0.45212) (xy -4.25958 -0.45212) (xy -4.25958 0.82296) (xy -4.0386 0.82296) (xy -4.0386 -0.45212)) (layer "B.Cu")
   (width 0.01) (fill solid)))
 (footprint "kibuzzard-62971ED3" (layer "B.Cu") (at 129.8 75.05 180)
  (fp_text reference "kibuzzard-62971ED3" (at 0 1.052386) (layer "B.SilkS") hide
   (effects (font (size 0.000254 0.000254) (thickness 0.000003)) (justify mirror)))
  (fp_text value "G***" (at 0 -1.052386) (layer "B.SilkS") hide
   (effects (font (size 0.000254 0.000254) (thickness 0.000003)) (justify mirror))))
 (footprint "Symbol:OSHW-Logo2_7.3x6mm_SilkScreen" (layer "B.Cu") (at 138.2 80.9 180)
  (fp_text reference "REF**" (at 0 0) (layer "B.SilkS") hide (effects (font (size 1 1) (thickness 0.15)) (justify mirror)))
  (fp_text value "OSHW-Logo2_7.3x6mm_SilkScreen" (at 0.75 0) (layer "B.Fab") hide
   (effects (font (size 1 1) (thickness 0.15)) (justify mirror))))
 (gr_line (start 122.5 73) (end 122.5 92) (layer "Edge.Cuts") (width 0.05))
 (gr_line (start 122.5 92) (end 147.5 92) (layer "Edge.Cuts") (width 0.05))
 (gr_line (start 147.5 73) (end 122.5 73) (layer "Edge.Cuts") (width 0.05))
 (gr_line (start 147.5 92) (end 147.5 73) (layer "Edge.Cuts") (width 0.05))
 (segment (start 131.07 80.26) (end 131.07 80.07) (width 0.8) (layer "F.Cu") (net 4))
 (segment (start 132.42 84.2) (end 131.07 82.85) (width 0.8) (layer "F.Cu") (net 4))
 (segment (start 131.07 82.85) (end 131.07 80.26) (width 0.8) (layer "F.Cu") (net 4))
 (segment (start 131.07 80.07) (end 127.26 76.26) (width 0.8) (layer "F.Cu") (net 4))
 (segment (start 132.5 86.58) (end 132.42 86.5) (width 0.8) (layer "F.Cu") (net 4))
 (segment (start 132.42 86.5) (end 132.42 84.2) (width 0.8) (layer "F.Cu") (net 4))
 (segment (start 125.56 80.26) (end 125 79.7) (width 0.8) (layer "F.Cu") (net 2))
 (segment (start 142.5 74.5) (end 142.5 76.26) (width 0.8) (layer "F.Cu") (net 2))
 (segment (start 144.5 76.56) (end 144.5 82) (width 0.8) (layer "F.Cu") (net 2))
 (segment (start 142.5 76.26) (end 144.2 76.26) (width 0.8) (layer "F.Cu") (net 2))
 (segment (start 139.25 84.75) (end 137.5 86.5) (width 0.8) (layer "F.Cu") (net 2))
 (segment (start 125 75) (end 126 74) (width 0.8) (layer "F.Cu") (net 2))
 (segment (start 144.2 76.26) (end 144.5 76.56) (width 0.8) (layer "F.Cu") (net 2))
 (segment (start 125 79.7) (end 125 75) (width 0.8) (layer "F.Cu") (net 2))
 (segment (start 126 74) (end 142 74) (width 0.8) (layer "F.Cu") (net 2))
 (segment (start 144 82.5) (end 141.5 82.5) (width 0.8) (layer "F.Cu") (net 2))
 (segment (start 141.5 82.5) (end 139.25 84.75) (width 0.8) (layer "F.Cu") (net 2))
 (segment (start 127.26 80.26) (end 125.56 80.26) (width 0.8) (layer "F.Cu") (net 2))
 (segment (start 142 74) (end 142.5 74.5) (width 0.8) (layer "F.Cu") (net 2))
 (segment (start 144.5 82) (end 144 82.5) (width 0.8) (layer "F.Cu") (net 2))
 (segment (start 134.88 80.26) (end 134.88 80.07) (width 0.8) (layer "F.Cu") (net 5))
 (segment (start 134.88 80.07) (end 131.07 76.26) (width 0.8) (layer "F.Cu") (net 5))
 (segment (start 142.5 80.26) (end 142.5 80.07) (width 0.8) (layer "F.Cu") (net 1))
 (segment (start 142.5 80.07) (end 138.69 76.26) (width 0.8) (layer "F.Cu") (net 1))
 (segment (start 138.69 80.07) (end 134.88 76.26) (width 0.8) (layer "F.Cu") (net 3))
 (segment (start 138.69 80.26) (end 138.69 80.07) (width 0.8) (layer "F.Cu") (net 3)))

